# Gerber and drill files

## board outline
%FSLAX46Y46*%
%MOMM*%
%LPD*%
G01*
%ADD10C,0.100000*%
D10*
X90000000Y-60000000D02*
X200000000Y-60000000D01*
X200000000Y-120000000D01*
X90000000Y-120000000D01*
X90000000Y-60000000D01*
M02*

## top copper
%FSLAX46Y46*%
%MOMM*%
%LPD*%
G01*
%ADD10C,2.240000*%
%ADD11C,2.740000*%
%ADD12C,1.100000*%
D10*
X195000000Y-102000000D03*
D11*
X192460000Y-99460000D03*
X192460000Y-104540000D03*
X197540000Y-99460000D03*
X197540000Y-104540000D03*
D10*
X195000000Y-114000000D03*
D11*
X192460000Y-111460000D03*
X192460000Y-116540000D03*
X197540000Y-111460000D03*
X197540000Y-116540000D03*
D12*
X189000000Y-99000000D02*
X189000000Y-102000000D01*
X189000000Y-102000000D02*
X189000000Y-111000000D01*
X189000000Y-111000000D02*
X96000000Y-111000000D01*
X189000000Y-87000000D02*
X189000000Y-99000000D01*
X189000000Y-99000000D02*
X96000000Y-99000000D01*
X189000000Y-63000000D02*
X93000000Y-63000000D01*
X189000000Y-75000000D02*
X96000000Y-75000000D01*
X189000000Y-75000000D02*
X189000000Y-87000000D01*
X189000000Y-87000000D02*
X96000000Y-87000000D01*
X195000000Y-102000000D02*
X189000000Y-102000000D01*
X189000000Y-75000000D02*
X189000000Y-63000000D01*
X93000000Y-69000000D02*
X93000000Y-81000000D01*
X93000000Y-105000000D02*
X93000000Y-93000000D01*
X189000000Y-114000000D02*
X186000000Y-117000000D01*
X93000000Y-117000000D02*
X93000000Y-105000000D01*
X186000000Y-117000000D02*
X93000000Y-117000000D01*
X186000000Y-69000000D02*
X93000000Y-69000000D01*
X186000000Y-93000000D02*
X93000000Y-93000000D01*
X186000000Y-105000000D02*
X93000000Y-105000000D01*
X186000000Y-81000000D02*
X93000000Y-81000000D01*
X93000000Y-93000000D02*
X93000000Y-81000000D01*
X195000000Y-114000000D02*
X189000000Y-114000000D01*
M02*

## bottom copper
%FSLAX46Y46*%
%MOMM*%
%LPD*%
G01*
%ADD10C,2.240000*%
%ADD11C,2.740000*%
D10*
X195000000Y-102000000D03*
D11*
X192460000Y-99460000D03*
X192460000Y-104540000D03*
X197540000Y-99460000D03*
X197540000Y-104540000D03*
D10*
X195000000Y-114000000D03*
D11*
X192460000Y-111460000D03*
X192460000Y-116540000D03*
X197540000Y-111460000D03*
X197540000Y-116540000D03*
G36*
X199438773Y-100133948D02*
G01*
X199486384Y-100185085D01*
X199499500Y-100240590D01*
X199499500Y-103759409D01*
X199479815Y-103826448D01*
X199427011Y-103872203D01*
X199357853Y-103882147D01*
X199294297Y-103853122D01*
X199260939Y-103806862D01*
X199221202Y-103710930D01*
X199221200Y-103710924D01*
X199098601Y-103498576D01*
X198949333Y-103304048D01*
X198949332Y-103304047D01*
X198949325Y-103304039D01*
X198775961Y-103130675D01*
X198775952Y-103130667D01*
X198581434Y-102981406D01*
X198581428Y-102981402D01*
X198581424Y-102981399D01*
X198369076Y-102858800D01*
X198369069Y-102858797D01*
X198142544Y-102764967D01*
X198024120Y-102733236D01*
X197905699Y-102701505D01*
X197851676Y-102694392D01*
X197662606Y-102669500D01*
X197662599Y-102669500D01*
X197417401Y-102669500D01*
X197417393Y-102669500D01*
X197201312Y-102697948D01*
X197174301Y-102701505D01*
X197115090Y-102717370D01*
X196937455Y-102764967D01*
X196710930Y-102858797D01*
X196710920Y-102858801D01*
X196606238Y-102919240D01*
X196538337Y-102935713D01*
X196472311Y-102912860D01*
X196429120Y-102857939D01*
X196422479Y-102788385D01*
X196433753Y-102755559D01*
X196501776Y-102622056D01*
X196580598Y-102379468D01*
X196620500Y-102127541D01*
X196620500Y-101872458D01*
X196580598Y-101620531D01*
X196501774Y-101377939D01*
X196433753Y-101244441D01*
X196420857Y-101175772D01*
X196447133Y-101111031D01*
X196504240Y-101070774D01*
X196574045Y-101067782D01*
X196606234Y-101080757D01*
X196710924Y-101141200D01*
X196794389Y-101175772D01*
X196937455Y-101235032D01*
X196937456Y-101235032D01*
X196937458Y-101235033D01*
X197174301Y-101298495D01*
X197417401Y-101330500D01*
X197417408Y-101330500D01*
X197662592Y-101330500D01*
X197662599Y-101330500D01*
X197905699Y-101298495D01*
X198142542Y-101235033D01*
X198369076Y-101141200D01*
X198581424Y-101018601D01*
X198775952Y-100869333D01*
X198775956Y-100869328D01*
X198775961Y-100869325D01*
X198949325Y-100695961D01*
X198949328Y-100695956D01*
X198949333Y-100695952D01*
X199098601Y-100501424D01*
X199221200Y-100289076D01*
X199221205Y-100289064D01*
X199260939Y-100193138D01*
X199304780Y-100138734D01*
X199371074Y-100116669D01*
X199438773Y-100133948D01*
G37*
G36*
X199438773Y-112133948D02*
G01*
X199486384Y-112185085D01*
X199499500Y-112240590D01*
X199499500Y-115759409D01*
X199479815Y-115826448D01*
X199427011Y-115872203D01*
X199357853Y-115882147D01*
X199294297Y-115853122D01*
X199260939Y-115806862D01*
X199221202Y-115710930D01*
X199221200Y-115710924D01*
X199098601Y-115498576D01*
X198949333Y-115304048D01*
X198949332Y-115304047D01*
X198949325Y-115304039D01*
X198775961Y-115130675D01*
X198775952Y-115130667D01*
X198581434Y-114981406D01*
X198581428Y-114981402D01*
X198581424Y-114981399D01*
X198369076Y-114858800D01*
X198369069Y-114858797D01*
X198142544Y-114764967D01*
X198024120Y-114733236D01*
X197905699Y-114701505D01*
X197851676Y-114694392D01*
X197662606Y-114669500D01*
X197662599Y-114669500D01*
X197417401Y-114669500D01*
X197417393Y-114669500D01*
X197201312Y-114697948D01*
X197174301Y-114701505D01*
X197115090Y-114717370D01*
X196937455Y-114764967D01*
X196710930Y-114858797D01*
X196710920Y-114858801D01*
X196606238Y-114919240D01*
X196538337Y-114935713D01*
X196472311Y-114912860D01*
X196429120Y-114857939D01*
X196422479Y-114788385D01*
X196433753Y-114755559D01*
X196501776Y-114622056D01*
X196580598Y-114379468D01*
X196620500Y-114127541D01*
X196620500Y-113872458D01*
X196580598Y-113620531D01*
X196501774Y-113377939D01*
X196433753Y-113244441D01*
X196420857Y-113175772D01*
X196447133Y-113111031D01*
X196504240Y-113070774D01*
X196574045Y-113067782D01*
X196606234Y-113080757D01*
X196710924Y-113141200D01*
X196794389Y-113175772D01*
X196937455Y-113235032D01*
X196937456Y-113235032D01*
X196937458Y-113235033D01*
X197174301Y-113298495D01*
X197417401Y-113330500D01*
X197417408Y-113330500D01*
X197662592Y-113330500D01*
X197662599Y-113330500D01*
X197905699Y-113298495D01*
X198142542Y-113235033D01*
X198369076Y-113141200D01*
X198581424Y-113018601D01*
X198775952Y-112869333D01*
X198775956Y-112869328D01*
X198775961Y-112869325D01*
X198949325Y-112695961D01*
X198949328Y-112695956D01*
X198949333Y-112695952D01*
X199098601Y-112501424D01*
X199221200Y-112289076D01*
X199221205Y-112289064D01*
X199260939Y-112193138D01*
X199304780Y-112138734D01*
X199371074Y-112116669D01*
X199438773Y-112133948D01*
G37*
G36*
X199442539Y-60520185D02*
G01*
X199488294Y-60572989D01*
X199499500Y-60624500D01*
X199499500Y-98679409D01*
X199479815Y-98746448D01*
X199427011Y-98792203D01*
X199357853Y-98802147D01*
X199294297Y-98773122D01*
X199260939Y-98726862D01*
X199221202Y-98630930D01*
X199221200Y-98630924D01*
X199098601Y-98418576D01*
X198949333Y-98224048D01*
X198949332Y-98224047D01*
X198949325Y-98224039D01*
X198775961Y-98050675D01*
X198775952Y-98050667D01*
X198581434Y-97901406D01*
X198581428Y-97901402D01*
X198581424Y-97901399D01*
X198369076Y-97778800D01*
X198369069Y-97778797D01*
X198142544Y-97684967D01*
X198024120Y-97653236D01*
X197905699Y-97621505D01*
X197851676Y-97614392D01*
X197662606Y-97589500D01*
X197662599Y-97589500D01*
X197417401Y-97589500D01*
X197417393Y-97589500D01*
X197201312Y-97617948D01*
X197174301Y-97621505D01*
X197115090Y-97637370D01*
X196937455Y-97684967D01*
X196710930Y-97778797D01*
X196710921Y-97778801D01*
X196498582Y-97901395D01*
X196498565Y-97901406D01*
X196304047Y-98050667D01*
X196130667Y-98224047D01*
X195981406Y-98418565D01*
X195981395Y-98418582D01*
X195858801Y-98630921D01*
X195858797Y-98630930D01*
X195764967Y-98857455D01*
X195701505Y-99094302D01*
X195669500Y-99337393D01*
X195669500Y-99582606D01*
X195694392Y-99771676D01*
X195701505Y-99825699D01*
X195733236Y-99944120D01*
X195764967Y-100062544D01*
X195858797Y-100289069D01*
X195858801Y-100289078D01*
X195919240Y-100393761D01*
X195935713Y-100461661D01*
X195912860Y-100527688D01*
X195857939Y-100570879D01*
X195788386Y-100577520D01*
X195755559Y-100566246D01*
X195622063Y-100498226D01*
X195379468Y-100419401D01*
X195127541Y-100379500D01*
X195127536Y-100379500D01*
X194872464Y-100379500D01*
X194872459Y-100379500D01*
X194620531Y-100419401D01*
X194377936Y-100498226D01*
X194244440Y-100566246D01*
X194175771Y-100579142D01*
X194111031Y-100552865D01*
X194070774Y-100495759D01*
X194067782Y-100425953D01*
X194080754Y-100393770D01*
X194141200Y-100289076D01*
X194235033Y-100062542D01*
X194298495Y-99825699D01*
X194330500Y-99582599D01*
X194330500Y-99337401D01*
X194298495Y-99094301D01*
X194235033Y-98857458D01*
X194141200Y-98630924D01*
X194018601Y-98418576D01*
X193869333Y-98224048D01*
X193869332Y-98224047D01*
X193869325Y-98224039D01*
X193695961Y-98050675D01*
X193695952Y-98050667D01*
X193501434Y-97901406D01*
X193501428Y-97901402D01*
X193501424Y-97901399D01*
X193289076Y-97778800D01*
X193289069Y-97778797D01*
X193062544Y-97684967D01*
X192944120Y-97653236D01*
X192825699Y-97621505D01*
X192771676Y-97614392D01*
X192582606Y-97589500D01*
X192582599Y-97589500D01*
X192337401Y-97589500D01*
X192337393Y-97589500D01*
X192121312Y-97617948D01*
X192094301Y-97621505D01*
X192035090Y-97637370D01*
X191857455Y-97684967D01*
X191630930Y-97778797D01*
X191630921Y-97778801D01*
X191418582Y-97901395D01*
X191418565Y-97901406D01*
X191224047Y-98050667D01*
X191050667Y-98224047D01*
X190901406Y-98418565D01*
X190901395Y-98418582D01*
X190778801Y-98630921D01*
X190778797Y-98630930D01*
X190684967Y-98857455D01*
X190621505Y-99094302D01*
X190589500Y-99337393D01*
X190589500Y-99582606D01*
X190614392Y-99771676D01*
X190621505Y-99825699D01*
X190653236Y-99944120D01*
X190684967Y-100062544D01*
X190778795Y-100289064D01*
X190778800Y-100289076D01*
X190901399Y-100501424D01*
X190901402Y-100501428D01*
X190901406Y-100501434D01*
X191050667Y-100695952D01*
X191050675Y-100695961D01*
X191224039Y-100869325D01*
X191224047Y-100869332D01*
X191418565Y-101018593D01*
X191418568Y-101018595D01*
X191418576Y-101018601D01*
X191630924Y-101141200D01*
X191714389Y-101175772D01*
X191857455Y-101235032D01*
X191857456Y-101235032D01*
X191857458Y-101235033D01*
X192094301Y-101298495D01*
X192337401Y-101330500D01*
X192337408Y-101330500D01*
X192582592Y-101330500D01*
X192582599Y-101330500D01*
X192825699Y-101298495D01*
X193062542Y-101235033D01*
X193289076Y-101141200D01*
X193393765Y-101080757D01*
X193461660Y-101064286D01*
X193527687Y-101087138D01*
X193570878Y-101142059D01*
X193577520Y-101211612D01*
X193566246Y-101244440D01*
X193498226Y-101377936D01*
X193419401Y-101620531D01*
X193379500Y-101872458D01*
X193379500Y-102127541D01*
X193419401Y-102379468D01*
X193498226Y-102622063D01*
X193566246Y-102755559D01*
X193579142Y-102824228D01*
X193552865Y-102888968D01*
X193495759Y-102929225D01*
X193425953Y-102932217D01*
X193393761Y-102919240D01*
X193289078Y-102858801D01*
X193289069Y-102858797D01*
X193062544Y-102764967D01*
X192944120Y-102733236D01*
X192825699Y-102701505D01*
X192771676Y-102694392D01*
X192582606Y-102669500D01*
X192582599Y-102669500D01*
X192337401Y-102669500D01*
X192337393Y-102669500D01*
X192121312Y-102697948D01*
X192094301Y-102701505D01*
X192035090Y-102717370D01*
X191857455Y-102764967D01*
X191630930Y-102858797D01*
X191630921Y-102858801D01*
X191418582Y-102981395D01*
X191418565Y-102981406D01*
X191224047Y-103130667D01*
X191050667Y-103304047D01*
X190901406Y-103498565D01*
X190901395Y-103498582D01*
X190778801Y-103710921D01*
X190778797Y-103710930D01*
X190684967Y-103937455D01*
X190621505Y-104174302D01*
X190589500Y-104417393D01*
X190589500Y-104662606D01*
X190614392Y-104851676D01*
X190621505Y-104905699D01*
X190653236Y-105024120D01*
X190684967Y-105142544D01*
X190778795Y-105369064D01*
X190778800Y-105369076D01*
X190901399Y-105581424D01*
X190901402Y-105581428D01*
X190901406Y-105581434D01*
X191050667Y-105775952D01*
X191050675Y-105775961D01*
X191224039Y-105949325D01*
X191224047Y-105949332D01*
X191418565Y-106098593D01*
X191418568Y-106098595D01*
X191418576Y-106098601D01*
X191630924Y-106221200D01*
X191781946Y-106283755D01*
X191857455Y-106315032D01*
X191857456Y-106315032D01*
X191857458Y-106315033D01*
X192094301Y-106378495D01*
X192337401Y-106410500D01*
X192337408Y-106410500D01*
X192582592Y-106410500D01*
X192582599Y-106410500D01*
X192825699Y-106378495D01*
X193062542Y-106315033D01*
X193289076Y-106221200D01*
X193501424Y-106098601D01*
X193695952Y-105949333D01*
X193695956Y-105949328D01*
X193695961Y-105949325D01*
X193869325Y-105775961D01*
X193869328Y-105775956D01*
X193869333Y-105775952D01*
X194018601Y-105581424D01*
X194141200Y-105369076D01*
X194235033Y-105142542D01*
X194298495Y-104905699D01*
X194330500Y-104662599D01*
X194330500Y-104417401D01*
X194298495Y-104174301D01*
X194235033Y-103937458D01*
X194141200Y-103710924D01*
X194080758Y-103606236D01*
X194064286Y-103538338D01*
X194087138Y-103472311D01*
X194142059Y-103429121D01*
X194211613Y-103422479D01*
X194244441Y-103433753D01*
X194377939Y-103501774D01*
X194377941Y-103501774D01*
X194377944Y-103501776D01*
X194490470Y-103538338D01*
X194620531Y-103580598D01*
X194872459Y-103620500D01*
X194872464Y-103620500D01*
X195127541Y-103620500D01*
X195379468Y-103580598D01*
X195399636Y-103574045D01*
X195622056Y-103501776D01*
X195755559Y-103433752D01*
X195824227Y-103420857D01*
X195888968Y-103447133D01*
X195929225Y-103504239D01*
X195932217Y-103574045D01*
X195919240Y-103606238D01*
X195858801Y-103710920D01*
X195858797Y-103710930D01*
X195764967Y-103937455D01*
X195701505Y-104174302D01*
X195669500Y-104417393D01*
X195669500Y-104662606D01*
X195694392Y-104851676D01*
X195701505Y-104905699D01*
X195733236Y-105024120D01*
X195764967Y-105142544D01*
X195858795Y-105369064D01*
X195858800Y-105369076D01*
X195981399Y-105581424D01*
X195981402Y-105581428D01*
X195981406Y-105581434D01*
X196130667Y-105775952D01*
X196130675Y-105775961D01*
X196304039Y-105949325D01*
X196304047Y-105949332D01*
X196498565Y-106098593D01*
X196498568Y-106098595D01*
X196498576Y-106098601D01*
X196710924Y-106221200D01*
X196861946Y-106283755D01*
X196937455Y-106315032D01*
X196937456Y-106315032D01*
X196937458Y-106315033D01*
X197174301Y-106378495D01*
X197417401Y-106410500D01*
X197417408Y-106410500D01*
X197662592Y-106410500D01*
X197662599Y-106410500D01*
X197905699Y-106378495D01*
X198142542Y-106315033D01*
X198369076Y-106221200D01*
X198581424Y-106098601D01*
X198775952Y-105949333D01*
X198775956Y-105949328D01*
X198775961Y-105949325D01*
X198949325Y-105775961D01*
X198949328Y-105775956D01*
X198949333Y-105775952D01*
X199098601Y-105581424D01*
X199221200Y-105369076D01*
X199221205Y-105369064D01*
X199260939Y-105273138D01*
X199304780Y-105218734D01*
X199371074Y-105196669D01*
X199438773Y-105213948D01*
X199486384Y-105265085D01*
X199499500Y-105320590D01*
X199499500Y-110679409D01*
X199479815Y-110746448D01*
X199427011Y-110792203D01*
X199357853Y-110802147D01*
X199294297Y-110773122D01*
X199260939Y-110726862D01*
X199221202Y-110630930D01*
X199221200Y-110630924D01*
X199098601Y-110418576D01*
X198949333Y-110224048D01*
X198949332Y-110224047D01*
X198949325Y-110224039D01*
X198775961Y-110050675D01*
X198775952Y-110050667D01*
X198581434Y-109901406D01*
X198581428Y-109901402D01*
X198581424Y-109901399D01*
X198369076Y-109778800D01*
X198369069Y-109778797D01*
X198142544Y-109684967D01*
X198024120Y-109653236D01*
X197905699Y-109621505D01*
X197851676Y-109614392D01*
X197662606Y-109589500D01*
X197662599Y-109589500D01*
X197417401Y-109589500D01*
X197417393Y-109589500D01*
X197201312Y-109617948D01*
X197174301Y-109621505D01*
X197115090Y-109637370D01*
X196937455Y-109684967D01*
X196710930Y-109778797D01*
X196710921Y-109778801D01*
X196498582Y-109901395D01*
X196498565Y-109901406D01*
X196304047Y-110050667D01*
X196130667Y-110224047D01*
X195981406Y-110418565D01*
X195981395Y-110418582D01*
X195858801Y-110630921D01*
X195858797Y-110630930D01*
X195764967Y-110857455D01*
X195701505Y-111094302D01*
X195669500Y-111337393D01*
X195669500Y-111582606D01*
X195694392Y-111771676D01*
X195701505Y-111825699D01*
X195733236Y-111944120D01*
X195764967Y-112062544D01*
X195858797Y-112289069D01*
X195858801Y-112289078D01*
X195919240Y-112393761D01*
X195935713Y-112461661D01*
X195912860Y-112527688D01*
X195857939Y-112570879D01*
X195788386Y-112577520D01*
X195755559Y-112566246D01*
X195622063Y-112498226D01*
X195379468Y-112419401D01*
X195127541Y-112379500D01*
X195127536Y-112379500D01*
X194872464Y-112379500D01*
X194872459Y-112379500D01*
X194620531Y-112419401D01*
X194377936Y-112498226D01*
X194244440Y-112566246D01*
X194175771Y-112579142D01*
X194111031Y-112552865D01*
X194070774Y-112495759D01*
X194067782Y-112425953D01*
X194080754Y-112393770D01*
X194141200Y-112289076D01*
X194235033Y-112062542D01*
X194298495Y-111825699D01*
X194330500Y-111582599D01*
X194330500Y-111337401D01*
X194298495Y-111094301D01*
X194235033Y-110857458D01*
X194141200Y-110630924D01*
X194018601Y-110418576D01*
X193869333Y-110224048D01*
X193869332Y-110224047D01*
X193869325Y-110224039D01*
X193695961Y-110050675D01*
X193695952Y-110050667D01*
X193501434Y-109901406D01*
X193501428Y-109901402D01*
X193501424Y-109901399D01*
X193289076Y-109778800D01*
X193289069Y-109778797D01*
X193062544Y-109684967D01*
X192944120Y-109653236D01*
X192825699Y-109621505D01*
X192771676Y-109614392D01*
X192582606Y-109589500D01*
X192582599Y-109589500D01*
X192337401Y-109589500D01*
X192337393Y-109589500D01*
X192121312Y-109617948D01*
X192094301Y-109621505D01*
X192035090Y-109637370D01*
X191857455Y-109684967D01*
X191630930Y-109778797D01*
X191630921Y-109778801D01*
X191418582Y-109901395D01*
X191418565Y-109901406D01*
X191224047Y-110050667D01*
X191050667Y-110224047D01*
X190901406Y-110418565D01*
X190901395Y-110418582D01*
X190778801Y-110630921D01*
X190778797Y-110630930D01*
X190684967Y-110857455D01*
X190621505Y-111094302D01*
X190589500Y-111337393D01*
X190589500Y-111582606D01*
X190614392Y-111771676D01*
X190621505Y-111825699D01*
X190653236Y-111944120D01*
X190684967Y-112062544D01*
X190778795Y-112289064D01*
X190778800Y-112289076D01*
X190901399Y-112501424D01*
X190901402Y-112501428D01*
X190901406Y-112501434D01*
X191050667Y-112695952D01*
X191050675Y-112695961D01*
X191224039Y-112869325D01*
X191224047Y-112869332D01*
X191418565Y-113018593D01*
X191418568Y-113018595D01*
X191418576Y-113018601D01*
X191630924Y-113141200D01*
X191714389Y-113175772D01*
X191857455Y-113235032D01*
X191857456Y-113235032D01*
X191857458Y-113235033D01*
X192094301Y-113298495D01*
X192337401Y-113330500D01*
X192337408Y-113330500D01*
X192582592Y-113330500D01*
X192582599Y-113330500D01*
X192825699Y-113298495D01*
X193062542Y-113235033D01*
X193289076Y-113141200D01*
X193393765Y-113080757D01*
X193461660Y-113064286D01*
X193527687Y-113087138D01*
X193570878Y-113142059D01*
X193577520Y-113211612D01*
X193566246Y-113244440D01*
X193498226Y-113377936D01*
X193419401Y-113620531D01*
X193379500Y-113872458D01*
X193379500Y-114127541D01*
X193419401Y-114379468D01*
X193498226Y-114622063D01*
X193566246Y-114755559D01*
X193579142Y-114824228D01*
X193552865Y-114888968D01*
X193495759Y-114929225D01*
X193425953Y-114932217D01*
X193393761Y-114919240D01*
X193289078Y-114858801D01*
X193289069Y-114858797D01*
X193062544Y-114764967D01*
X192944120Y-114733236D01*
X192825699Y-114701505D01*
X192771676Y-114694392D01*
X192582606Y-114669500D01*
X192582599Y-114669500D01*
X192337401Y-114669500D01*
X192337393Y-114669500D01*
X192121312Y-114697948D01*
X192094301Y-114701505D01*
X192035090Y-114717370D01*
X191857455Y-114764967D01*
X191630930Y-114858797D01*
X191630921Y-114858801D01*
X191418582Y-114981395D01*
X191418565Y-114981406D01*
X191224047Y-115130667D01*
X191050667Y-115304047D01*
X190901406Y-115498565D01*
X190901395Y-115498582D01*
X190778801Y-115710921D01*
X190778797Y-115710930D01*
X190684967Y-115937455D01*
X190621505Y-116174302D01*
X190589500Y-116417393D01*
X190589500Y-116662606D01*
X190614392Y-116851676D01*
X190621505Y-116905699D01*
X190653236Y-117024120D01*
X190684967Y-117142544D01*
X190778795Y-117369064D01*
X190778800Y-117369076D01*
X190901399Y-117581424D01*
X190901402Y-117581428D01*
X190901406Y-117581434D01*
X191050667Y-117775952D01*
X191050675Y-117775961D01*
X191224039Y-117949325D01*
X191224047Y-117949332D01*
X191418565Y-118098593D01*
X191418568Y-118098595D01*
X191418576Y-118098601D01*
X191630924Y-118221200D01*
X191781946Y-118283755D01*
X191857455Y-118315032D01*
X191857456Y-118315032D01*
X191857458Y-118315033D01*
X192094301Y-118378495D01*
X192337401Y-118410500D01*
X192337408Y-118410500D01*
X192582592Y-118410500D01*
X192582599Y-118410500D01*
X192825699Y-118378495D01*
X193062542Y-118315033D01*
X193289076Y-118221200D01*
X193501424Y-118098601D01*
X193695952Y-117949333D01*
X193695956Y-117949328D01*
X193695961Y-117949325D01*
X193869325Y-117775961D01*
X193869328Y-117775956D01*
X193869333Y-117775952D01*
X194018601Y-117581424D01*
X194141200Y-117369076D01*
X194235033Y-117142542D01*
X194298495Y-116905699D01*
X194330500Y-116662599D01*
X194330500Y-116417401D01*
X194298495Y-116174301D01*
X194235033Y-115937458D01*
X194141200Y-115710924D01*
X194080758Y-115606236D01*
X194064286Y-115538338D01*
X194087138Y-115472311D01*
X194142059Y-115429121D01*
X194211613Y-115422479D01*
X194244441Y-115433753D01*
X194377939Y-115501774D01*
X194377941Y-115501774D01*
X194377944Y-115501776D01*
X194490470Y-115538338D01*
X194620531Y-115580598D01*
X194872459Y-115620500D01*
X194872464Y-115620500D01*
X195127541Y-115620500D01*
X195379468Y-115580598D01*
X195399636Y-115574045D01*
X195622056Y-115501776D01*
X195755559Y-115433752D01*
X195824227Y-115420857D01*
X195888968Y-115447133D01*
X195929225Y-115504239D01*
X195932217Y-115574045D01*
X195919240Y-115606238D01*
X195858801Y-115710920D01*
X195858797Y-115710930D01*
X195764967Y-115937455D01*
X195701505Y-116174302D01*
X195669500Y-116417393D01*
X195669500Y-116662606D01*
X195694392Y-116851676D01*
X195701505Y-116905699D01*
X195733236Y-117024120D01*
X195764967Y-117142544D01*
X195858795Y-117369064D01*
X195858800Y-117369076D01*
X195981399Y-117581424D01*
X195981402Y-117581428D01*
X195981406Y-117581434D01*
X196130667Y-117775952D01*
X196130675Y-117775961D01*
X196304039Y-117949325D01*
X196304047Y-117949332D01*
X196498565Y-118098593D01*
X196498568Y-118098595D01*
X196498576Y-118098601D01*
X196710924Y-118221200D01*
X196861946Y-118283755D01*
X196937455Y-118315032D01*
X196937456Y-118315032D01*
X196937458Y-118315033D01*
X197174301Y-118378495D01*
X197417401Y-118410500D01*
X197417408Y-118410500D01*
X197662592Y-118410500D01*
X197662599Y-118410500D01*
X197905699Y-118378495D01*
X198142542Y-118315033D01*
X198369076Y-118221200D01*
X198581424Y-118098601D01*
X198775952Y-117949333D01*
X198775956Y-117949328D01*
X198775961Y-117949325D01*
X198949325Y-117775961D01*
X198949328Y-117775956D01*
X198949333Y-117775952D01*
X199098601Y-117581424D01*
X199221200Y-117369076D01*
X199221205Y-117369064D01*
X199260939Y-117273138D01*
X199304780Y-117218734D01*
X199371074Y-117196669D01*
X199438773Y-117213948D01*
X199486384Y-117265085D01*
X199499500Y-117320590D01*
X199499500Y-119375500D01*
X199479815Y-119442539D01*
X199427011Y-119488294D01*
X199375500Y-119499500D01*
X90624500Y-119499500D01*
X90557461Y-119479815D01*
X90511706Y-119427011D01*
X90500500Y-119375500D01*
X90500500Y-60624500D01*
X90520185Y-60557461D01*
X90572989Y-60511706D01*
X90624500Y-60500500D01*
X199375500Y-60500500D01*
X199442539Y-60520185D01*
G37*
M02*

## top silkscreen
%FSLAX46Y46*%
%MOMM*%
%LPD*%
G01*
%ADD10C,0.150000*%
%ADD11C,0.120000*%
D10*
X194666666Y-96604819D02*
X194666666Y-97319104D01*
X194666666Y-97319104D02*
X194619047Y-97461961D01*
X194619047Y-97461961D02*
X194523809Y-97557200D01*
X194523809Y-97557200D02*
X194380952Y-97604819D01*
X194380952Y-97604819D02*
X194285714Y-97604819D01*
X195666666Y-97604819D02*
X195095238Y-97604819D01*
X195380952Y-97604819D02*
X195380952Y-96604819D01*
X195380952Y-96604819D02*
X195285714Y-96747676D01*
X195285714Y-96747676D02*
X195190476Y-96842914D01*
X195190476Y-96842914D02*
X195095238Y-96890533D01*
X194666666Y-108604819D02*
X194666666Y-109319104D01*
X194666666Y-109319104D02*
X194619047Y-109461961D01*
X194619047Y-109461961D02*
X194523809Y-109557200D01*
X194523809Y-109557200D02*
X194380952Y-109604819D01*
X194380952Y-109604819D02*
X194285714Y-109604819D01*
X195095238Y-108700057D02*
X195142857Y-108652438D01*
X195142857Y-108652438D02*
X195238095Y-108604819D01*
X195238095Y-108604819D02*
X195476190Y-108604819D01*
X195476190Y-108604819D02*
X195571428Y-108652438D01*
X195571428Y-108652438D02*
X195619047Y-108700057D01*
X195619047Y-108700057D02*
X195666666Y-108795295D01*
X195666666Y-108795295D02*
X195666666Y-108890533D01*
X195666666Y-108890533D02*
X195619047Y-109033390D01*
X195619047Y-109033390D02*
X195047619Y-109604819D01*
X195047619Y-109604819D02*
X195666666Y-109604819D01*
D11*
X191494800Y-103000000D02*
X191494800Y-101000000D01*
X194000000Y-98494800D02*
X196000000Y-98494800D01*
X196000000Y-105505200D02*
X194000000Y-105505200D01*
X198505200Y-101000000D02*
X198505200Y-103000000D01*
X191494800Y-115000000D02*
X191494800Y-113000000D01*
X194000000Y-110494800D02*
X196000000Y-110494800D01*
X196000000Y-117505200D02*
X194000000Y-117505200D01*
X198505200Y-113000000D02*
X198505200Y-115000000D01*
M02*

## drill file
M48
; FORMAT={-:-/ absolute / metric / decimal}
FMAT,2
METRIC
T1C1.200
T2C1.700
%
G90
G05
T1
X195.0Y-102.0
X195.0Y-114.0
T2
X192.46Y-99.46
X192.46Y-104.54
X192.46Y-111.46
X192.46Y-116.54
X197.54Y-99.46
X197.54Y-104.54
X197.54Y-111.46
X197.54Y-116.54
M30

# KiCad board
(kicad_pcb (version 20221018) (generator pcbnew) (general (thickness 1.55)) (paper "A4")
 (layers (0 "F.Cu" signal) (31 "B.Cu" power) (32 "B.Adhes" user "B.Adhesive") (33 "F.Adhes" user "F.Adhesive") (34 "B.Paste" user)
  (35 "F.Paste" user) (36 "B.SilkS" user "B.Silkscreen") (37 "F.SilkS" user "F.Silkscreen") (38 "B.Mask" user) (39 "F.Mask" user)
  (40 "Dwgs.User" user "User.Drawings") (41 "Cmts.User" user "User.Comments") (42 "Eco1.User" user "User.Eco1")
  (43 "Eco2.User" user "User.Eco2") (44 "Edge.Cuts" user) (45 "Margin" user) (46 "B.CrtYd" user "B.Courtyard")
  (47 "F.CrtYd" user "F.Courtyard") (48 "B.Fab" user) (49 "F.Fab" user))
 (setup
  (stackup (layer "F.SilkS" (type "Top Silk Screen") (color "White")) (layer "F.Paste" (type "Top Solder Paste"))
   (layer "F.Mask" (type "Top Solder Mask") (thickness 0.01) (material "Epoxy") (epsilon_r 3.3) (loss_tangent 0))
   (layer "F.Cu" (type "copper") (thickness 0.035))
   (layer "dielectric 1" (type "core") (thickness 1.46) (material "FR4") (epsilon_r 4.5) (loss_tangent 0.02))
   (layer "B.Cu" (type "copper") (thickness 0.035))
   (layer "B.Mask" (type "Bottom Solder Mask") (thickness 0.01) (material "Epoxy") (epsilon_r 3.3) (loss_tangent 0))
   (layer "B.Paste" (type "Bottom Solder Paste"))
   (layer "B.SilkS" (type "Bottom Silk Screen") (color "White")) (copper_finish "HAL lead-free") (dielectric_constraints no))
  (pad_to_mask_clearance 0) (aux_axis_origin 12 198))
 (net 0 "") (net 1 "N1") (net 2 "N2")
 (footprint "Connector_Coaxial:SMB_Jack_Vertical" (layer "F.Cu") (at 195 102)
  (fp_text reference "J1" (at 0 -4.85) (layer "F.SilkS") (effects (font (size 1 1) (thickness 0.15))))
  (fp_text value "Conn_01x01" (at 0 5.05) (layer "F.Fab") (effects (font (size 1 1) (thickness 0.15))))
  (fp_line (start -3.5052 1) (end -3.5052 -1) (stroke (width 0.12) (type solid)) (layer "F.SilkS"))
  (fp_line (start -1 -3.5052) (end 1 -3.5052) (stroke (width 0.12) (type solid)) (layer "F.SilkS"))
  (fp_line (start 1 3.5052) (end -1 3.5052) (stroke (width 0.12) (type solid)) (layer "F.SilkS"))
  (fp_line (start 3.5052 -1) (end 3.5052 1) (stroke (width 0.12) (type solid)) (layer "F.SilkS"))
  (pad "1" thru_hole circle (at 0 0) (size 2.24 2.24) (drill 1.2) (layers "*.Cu" "*.Mask") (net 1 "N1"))
  (pad "2" thru_hole circle (at -2.54 -2.54) (size 2.74 2.74) (drill 1.7) (layers "*.Cu" "*.Mask"))
  (pad "2" thru_hole circle (at -2.54 2.54) (size 2.74 2.74) (drill 1.7) (layers "*.Cu" "*.Mask"))
  (pad "2" thru_hole circle (at 2.54 -2.54) (size 2.74 2.74) (drill 1.7) (layers "*.Cu" "*.Mask"))
  (pad "2" thru_hole circle (at 2.54 2.54) (size 2.74 2.74) (drill 1.7) (layers "*.Cu" "*.Mask")))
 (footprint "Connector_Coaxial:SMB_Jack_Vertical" (layer "F.Cu") (at 195 114)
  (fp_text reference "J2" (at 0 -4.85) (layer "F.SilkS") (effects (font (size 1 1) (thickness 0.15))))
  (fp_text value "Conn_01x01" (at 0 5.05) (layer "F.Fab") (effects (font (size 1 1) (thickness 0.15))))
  (fp_line (start -3.5052 1) (end -3.5052 -1) (stroke (width 0.12) (type solid)) (layer "F.SilkS"))
  (fp_line (start -1 -3.5052) (end 1 -3.5052) (stroke (width 0.12) (type solid)) (layer "F.SilkS"))
  (fp_line (start 1 3.5052) (end -1 3.5052) (stroke (width 0.12) (type solid)) (layer "F.SilkS"))
  (fp_line (start 3.5052 -1) (end 3.5052 1) (stroke (width 0.12) (type solid)) (layer "F.SilkS"))
  (pad "1" thru_hole circle (at 0 0) (size 2.24 2.24) (drill 1.2) (layers "*.Cu" "*.Mask") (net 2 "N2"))
  (pad "2" thru_hole circle (at -2.54 -2.54) (size 2.74 2.74) (drill 1.7) (layers "*.Cu" "*.Mask"))
  (pad "2" thru_hole circle (at -2.54 2.54) (size 2.74 2.74) (drill 1.7) (layers "*.Cu" "*.Mask"))
  (pad "2" thru_hole circle (at 2.54 -2.54) (size 2.74 2.74) (drill 1.7) (layers "*.Cu" "*.Mask"))
  (pad "2" thru_hole circle (at 2.54 2.54) (size 2.74 2.74) (drill 1.7) (layers "*.Cu" "*.Mask")))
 (gr_rect (start 90 60) (end 200 120) (stroke (width 0.1) (type default)) (fill none) (layer "Edge.Cuts"))
 (segment (start 189 99) (end 189 102) (width 1.1) (layer "F.Cu") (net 1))
 (segment (start 189 102) (end 189 111) (width 1.1) (layer "F.Cu") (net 1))
 (segment (start 189 111) (end 96 111) (width 1.1) (layer "F.Cu") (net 1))
 (segment (start 189 87) (end 189 99) (width 1.1) (layer "F.Cu") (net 1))
 (segment (start 189 99) (end 96 99) (width 1.1) (layer "F.Cu") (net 1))
 (segment (start 189 63) (end 93 63) (width 1.1) (layer "F.Cu") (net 1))
 (segment (start 189 75) (end 96 75) (width 1.1) (layer "F.Cu") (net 1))
 (segment (start 189 75) (end 189 87) (width 1.1) (layer "F.Cu") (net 1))
 (segment (start 189 87) (end 96 87) (width 1.1) (layer "F.Cu") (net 1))
 (segment (start 195 102) (end 189 102) (width 1.1) (layer "F.Cu") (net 1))
 (segment (start 189 75) (end 189 63) (width 1.1) (layer "F.Cu") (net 1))
 (segment (start 93 69) (end 93 81) (width 1.1) (layer "F.Cu") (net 2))
 (segment (start 93 105) (end 93 93) (width 1.1) (layer "F.Cu") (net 2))
 (segment (start 189 114) (end 186 117) (width 1.1) (layer "F.Cu") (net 2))
 (segment (start 93 117) (end 93 105) (width 1.1) (layer "F.Cu") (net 2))
 (segment (start 186 117) (end 93 117) (width 1.1) (layer "F.Cu") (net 2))
 (segment (start 186 69) (end 93 69) (width 1.1) (layer "F.Cu") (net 2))
 (segment (start 186 93) (end 93 93) (width 1.1) (layer "F.Cu") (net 2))
 (segment (start 186 105) (end 93 105) (width 1.1) (layer "F.Cu") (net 2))
 (segment (start 186 81) (end 93 81) (width 1.1) (layer "F.Cu") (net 2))
 (segment (start 93 93) (end 93 81) (width 1.1) (layer "F.Cu") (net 2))
 (segment (start 195 114) (end 189 114) (width 1.1) (layer "F.Cu") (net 2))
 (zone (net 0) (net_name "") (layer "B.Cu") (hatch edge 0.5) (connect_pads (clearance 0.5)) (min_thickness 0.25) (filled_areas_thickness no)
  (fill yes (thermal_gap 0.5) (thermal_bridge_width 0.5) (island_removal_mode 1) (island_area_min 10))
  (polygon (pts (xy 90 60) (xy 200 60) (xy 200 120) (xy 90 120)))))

